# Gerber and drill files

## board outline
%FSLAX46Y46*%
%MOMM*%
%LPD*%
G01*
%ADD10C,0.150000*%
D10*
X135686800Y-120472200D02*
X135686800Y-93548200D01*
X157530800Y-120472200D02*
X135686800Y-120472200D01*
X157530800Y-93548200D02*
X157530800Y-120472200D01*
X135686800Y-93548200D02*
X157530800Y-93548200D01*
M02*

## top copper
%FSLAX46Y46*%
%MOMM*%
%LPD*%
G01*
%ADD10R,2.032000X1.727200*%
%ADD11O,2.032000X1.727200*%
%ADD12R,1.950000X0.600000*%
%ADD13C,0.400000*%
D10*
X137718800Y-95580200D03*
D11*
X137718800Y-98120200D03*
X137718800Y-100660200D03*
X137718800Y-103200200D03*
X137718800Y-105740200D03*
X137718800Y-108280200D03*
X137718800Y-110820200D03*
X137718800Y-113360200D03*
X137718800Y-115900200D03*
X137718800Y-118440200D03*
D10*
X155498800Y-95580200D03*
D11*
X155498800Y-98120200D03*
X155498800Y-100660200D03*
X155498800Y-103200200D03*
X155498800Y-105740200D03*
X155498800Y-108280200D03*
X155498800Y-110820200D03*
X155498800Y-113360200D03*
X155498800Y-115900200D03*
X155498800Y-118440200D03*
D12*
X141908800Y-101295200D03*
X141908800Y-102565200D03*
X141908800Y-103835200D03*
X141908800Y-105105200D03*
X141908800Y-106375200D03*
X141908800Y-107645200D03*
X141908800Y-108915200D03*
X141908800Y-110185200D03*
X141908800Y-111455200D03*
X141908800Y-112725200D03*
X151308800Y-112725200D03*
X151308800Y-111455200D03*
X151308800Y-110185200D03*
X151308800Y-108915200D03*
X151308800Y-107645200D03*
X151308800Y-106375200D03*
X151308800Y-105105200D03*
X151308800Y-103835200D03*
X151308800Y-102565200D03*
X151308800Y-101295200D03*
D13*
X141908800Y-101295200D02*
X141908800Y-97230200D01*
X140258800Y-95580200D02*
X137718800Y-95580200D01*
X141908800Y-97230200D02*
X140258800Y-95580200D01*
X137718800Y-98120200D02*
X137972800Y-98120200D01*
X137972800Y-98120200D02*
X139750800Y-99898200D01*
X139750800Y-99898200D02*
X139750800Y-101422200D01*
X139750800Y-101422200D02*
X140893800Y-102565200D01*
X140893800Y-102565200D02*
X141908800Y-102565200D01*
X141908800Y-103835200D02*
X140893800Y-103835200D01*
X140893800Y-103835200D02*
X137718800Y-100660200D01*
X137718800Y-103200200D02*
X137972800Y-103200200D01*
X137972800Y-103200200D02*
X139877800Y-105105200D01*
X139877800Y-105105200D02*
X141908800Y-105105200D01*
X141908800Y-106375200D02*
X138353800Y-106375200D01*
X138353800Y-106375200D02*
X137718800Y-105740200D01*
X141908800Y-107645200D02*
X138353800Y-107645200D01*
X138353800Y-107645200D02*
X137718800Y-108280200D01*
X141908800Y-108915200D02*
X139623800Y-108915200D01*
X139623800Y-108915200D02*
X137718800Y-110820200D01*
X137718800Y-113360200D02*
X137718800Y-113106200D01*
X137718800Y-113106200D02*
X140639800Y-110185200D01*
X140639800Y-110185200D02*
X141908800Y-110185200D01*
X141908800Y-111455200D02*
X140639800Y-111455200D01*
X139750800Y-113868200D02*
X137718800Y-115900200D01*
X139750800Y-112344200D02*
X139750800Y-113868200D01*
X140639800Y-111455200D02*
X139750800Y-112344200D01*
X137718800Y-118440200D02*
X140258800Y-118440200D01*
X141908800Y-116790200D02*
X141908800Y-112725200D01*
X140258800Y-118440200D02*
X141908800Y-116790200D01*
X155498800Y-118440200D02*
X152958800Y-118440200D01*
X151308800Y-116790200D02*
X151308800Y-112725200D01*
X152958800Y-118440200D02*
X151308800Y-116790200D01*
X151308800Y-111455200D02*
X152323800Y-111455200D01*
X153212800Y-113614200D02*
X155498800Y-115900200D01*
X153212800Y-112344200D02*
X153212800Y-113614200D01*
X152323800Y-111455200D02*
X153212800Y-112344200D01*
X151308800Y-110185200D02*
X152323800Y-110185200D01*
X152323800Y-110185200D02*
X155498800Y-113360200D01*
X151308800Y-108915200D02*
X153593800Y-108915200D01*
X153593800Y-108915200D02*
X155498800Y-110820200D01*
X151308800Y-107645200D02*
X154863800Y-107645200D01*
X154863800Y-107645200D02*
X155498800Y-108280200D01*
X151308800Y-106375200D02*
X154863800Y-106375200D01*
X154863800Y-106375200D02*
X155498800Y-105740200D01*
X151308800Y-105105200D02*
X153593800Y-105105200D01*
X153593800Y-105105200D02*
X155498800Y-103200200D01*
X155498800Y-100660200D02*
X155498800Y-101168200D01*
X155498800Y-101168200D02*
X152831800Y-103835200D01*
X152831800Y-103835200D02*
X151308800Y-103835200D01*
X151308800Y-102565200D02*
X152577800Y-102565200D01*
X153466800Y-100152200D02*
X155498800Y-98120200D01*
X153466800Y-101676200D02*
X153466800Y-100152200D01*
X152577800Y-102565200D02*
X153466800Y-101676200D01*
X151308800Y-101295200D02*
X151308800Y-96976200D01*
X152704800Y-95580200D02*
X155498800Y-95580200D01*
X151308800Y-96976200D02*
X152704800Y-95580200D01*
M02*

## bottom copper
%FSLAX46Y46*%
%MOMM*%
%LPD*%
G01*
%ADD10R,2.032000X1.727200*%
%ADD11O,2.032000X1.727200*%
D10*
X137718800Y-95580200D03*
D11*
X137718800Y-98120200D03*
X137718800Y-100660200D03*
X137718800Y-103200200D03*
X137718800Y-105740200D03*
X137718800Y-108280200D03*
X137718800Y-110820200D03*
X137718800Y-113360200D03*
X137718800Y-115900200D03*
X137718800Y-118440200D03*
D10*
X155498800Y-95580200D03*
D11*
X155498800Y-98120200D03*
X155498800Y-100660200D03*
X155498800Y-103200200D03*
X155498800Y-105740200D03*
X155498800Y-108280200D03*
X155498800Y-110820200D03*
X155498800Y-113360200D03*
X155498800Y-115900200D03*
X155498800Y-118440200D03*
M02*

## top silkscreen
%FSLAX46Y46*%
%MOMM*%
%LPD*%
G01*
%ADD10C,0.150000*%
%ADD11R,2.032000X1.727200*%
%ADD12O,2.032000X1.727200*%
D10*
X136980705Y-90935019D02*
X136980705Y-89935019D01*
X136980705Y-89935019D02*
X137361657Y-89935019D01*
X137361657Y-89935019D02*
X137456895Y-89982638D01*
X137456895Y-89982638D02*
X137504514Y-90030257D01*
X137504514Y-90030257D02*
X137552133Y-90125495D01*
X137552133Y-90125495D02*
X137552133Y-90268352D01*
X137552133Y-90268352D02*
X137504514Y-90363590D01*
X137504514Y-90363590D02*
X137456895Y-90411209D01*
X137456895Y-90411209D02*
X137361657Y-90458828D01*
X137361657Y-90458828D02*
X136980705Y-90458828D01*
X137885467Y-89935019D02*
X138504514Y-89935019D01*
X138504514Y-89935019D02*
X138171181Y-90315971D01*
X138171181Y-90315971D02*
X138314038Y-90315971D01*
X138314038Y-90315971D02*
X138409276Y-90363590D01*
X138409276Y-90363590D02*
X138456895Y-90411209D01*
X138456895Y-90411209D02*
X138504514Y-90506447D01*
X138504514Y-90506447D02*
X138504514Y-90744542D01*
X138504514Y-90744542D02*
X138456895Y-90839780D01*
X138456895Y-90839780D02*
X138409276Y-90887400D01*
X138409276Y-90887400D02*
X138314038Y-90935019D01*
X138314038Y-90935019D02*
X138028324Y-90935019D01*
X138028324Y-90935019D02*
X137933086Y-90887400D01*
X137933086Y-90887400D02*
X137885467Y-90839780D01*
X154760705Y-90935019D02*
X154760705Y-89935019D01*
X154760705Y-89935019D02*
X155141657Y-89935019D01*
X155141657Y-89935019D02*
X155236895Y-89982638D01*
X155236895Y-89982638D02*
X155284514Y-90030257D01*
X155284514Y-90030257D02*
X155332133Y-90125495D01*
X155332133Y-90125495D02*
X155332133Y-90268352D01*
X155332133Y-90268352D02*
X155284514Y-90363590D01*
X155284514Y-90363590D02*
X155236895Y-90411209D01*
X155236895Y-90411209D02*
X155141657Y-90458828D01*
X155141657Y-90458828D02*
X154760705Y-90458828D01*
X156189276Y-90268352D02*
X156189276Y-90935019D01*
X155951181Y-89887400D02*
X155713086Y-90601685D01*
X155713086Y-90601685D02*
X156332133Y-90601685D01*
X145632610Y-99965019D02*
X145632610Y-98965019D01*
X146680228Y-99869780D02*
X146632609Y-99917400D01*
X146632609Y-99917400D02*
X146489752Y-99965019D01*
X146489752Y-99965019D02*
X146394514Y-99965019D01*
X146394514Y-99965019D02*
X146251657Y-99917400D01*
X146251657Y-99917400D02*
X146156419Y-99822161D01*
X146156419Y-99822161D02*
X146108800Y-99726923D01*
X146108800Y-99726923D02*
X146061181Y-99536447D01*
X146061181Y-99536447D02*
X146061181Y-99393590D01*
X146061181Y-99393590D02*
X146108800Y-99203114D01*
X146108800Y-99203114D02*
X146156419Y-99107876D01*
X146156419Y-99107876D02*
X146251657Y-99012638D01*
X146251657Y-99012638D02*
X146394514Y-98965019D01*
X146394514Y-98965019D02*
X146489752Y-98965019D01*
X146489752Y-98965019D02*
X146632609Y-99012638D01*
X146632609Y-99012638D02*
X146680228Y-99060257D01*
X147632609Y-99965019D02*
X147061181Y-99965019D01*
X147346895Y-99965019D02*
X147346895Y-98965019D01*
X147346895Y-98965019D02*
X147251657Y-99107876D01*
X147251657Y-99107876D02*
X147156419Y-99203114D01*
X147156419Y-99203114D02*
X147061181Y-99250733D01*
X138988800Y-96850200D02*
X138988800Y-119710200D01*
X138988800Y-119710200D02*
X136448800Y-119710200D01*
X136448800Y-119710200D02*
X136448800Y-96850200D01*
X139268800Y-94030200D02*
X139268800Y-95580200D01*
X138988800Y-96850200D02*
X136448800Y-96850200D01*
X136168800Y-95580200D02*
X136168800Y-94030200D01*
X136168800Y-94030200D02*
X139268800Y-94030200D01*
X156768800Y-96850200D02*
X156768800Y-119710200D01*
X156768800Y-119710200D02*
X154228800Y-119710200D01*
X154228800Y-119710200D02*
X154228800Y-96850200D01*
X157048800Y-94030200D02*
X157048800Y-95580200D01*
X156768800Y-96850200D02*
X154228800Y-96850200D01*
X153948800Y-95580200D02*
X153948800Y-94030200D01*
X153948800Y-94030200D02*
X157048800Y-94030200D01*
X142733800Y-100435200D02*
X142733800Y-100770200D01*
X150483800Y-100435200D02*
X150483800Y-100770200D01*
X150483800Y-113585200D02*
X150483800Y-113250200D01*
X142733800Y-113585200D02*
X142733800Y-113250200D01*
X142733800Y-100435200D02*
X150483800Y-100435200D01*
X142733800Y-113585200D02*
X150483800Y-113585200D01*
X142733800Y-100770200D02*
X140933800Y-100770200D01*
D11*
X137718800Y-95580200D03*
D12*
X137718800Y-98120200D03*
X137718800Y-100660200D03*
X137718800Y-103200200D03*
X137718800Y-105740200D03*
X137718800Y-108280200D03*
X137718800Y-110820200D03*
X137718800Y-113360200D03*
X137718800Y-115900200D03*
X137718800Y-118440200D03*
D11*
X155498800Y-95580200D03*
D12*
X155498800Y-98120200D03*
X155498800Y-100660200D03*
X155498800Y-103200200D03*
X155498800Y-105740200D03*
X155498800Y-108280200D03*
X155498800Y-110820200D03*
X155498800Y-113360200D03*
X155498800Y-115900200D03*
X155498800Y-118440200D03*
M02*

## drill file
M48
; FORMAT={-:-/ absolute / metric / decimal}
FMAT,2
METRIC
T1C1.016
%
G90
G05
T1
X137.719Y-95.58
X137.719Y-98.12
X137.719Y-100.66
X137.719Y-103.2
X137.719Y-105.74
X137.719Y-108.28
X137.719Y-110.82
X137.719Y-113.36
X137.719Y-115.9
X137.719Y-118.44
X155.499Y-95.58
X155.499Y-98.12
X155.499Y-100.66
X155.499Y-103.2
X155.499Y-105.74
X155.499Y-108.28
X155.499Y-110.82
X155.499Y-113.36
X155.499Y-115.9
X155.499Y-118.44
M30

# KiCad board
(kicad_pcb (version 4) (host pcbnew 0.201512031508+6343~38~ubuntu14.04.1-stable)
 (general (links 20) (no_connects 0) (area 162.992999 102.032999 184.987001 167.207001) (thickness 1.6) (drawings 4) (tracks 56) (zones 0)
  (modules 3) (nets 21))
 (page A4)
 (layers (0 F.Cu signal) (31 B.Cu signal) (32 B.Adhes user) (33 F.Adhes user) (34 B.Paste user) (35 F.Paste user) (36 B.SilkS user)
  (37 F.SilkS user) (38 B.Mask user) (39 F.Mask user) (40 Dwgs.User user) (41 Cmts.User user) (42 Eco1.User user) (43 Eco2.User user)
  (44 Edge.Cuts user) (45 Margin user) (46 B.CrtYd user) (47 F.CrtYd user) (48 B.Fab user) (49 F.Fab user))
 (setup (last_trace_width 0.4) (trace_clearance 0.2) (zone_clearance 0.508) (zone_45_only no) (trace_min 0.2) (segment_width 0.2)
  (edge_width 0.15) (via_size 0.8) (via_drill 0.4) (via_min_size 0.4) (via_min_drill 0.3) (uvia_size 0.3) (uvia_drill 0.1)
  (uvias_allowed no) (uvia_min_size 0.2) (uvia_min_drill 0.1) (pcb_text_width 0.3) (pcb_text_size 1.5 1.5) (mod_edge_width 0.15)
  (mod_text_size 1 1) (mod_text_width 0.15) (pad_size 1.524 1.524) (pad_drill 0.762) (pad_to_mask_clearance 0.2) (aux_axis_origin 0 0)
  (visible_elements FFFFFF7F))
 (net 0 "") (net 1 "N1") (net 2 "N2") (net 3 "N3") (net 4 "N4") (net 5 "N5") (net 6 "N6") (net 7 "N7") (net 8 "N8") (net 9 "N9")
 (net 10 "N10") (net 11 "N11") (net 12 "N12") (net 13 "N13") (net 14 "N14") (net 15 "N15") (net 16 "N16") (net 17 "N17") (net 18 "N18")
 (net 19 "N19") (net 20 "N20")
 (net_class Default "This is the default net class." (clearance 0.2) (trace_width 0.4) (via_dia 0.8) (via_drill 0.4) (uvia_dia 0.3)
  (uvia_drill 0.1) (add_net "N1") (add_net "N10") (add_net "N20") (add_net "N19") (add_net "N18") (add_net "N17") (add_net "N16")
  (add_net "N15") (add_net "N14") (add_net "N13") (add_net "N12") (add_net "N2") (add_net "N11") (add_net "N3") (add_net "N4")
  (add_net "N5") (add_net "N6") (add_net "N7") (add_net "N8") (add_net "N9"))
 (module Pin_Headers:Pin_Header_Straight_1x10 (layer F.Cu) (at 137.7188 95.5802)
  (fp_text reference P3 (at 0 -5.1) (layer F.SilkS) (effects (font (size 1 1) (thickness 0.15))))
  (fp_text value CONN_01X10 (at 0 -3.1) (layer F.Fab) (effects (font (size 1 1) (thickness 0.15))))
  (fp_line (start 1.27 1.27) (end 1.27 24.13) (layer F.SilkS) (width 0.15))
  (fp_line (start 1.27 24.13) (end -1.27 24.13) (layer F.SilkS) (width 0.15))
  (fp_line (start -1.27 24.13) (end -1.27 1.27) (layer F.SilkS) (width 0.15))
  (fp_line (start 1.55 -1.55) (end 1.55 0) (layer F.SilkS) (width 0.15))
  (fp_line (start 1.27 1.27) (end -1.27 1.27) (layer F.SilkS) (width 0.15))
  (fp_line (start -1.55 0) (end -1.55 -1.55) (layer F.SilkS) (width 0.15))
  (fp_line (start -1.55 -1.55) (end 1.55 -1.55) (layer F.SilkS) (width 0.15))
  (pad 1 thru_hole rect (at 0 0) (size 2.032 1.7272) (drill 1.016) (layers *.Cu *.Mask F.SilkS) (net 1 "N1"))
  (pad 2 thru_hole oval (at 0 2.54) (size 2.032 1.7272) (drill 1.016) (layers *.Cu *.Mask F.SilkS) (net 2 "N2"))
  (pad 3 thru_hole oval (at 0 5.08) (size 2.032 1.7272) (drill 1.016) (layers *.Cu *.Mask F.SilkS) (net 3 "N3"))
  (pad 4 thru_hole oval (at 0 7.62) (size 2.032 1.7272) (drill 1.016) (layers *.Cu *.Mask F.SilkS) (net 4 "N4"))
  (pad 5 thru_hole oval (at 0 10.16) (size 2.032 1.7272) (drill 1.016) (layers *.Cu *.Mask F.SilkS) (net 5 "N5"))
  (pad 6 thru_hole oval (at 0 12.7) (size 2.032 1.7272) (drill 1.016) (layers *.Cu *.Mask F.SilkS) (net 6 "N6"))
  (pad 7 thru_hole oval (at 0 15.24) (size 2.032 1.7272) (drill 1.016) (layers *.Cu *.Mask F.SilkS) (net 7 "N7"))
  (pad 8 thru_hole oval (at 0 17.78) (size 2.032 1.7272) (drill 1.016) (layers *.Cu *.Mask F.SilkS) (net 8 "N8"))
  (pad 9 thru_hole oval (at 0 20.32) (size 2.032 1.7272) (drill 1.016) (layers *.Cu *.Mask F.SilkS) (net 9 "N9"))
  (pad 10 thru_hole oval (at 0 22.86) (size 2.032 1.7272) (drill 1.016) (layers *.Cu *.Mask F.SilkS) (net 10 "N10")))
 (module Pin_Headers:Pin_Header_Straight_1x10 (layer F.Cu) (at 155.4988 95.5802)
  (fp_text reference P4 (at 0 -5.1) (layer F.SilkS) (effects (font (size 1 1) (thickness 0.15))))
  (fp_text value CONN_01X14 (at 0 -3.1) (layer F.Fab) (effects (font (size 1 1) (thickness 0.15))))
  (fp_line (start 1.27 1.27) (end 1.27 24.13) (layer F.SilkS) (width 0.15))
  (fp_line (start 1.27 24.13) (end -1.27 24.13) (layer F.SilkS) (width 0.15))
  (fp_line (start -1.27 24.13) (end -1.27 1.27) (layer F.SilkS) (width 0.15))
  (fp_line (start 1.55 -1.55) (end 1.55 0) (layer F.SilkS) (width 0.15))
  (fp_line (start 1.27 1.27) (end -1.27 1.27) (layer F.SilkS) (width 0.15))
  (fp_line (start -1.55 0) (end -1.55 -1.55) (layer F.SilkS) (width 0.15))
  (fp_line (start -1.55 -1.55) (end 1.55 -1.55) (layer F.SilkS) (width 0.15))
  (pad 1 thru_hole rect (at 0 0) (size 2.032 1.7272) (drill 1.016) (layers *.Cu *.Mask F.SilkS) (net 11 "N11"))
  (pad 2 thru_hole oval (at 0 2.54) (size 2.032 1.7272) (drill 1.016) (layers *.Cu *.Mask F.SilkS) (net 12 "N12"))
  (pad 3 thru_hole oval (at 0 5.08) (size 2.032 1.7272) (drill 1.016) (layers *.Cu *.Mask F.SilkS) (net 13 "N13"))
  (pad 4 thru_hole oval (at 0 7.62) (size 2.032 1.7272) (drill 1.016) (layers *.Cu *.Mask F.SilkS) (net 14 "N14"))
  (pad 5 thru_hole oval (at 0 10.16) (size 2.032 1.7272) (drill 1.016) (layers *.Cu *.Mask F.SilkS) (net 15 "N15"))
  (pad 6 thru_hole oval (at 0 12.7) (size 2.032 1.7272) (drill 1.016) (layers *.Cu *.Mask F.SilkS) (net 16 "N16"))
  (pad 7 thru_hole oval (at 0 15.24) (size 2.032 1.7272) (drill 1.016) (layers *.Cu *.Mask F.SilkS) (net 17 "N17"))
  (pad 8 thru_hole oval (at 0 17.78) (size 2.032 1.7272) (drill 1.016) (layers *.Cu *.Mask F.SilkS) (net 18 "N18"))
  (pad 9 thru_hole oval (at 0 20.32) (size 2.032 1.7272) (drill 1.016) (layers *.Cu *.Mask F.SilkS) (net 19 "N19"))
  (pad 10 thru_hole oval (at 0 22.86) (size 2.032 1.7272) (drill 1.016) (layers *.Cu *.Mask F.SilkS) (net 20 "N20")))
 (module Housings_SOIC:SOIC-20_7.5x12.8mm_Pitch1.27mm (layer F.Cu) (at 146.6088 107.0102)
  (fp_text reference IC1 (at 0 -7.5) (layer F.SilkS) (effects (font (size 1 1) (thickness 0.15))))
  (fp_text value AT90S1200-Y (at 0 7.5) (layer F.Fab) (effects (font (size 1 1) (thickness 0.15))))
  (fp_line (start -3.875 -6.575) (end -3.875 -6.24) (layer F.SilkS) (width 0.15))
  (fp_line (start 3.875 -6.575) (end 3.875 -6.24) (layer F.SilkS) (width 0.15))
  (fp_line (start 3.875 6.575) (end 3.875 6.24) (layer F.SilkS) (width 0.15))
  (fp_line (start -3.875 6.575) (end -3.875 6.24) (layer F.SilkS) (width 0.15))
  (fp_line (start -3.875 -6.575) (end 3.875 -6.575) (layer F.SilkS) (width 0.15))
  (fp_line (start -3.875 6.575) (end 3.875 6.575) (layer F.SilkS) (width 0.15))
  (fp_line (start -3.875 -6.24) (end -5.675 -6.24) (layer F.SilkS) (width 0.15))
  (pad 1 smd rect (at -4.7 -5.715) (size 1.95 0.6) (layers F.Cu F.Paste F.Mask) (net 1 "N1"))
  (pad 2 smd rect (at -4.7 -4.445) (size 1.95 0.6) (layers F.Cu F.Paste F.Mask) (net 2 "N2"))
  (pad 3 smd rect (at -4.7 -3.175) (size 1.95 0.6) (layers F.Cu F.Paste F.Mask) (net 3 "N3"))
  (pad 4 smd rect (at -4.7 -1.905) (size 1.95 0.6) (layers F.Cu F.Paste F.Mask) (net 4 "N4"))
  (pad 5 smd rect (at -4.7 -0.635) (size 1.95 0.6) (layers F.Cu F.Paste F.Mask) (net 5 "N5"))
  (pad 6 smd rect (at -4.7 0.635) (size 1.95 0.6) (layers F.Cu F.Paste F.Mask) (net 6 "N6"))
  (pad 7 smd rect (at -4.7 1.905) (size 1.95 0.6) (layers F.Cu F.Paste F.Mask) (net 7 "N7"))
  (pad 8 smd rect (at -4.7 3.175) (size 1.95 0.6) (layers F.Cu F.Paste F.Mask) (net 8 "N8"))
  (pad 9 smd rect (at -4.7 4.445) (size 1.95 0.6) (layers F.Cu F.Paste F.Mask) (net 9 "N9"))
  (pad 10 smd rect (at -4.7 5.715) (size 1.95 0.6) (layers F.Cu F.Paste F.Mask) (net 10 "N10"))
  (pad 11 smd rect (at 4.7 5.715) (size 1.95 0.6) (layers F.Cu F.Paste F.Mask) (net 20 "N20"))
  (pad 12 smd rect (at 4.7 4.445) (size 1.95 0.6) (layers F.Cu F.Paste F.Mask) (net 19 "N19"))
  (pad 13 smd rect (at 4.7 3.175) (size 1.95 0.6) (layers F.Cu F.Paste F.Mask) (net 18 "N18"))
  (pad 14 smd rect (at 4.7 1.905) (size 1.95 0.6) (layers F.Cu F.Paste F.Mask) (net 17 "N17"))
  (pad 15 smd rect (at 4.7 0.635) (size 1.95 0.6) (layers F.Cu F.Paste F.Mask) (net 16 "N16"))
  (pad 16 smd rect (at 4.7 -0.635) (size 1.95 0.6) (layers F.Cu F.Paste F.Mask) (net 15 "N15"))
  (pad 17 smd rect (at 4.7 -1.905) (size 1.95 0.6) (layers F.Cu F.Paste F.Mask) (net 14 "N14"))
  (pad 18 smd rect (at 4.7 -3.175) (size 1.95 0.6) (layers F.Cu F.Paste F.Mask) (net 13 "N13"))
  (pad 19 smd rect (at 4.7 -4.445) (size 1.95 0.6) (layers F.Cu F.Paste F.Mask) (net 12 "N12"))
  (pad 20 smd rect (at 4.7 -5.715) (size 1.95 0.6) (layers F.Cu F.Paste F.Mask) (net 11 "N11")))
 (gr_line (start 135.6868 120.4722) (end 135.6868 93.5482) (angle 90) (layer Edge.Cuts) (width 0.15))
 (gr_line (start 157.5308 120.4722) (end 135.6868 120.4722) (angle 90) (layer Edge.Cuts) (width 0.15))
 (gr_line (start 157.5308 93.5482) (end 157.5308 120.4722) (angle 90) (layer Edge.Cuts) (width 0.15))
 (gr_line (start 135.6868 93.5482) (end 157.5308 93.5482) (angle 90) (layer Edge.Cuts) (width 0.15))
 (segment (start 141.9088 101.2952) (end 141.9088 97.2302) (width 0.4) (layer F.Cu) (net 1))
 (segment (start 140.2588 95.5802) (end 137.7188 95.5802) (width 0.4) (layer F.Cu) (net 1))
 (segment (start 141.9088 97.2302) (end 140.2588 95.5802) (width 0.4) (layer F.Cu) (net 1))
 (segment (start 137.7188 98.1202) (end 137.9728 98.1202) (width 0.4) (layer F.Cu) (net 2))
 (segment (start 137.9728 98.1202) (end 139.7508 99.8982) (width 0.4) (layer F.Cu) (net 2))
 (segment (start 139.7508 99.8982) (end 139.7508 101.4222) (width 0.4) (layer F.Cu) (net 2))
 (segment (start 139.7508 101.4222) (end 140.8938 102.5652) (width 0.4) (layer F.Cu) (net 2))
 (segment (start 140.8938 102.5652) (end 141.9088 102.5652) (width 0.4) (layer F.Cu) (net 2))
 (segment (start 141.9088 103.8352) (end 140.8938 103.8352) (width 0.4) (layer F.Cu) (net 3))
 (segment (start 140.8938 103.8352) (end 137.7188 100.6602) (width 0.4) (layer F.Cu) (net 3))
 (segment (start 137.7188 103.2002) (end 137.9728 103.2002) (width 0.4) (layer F.Cu) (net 4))
 (segment (start 137.9728 103.2002) (end 139.8778 105.1052) (width 0.4) (layer F.Cu) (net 4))
 (segment (start 139.8778 105.1052) (end 141.9088 105.1052) (width 0.4) (layer F.Cu) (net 4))
 (segment (start 141.9088 106.3752) (end 138.3538 106.3752) (width 0.4) (layer F.Cu) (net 5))
 (segment (start 138.3538 106.3752) (end 137.7188 105.7402) (width 0.4) (layer F.Cu) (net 5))
 (segment (start 141.9088 107.6452) (end 138.3538 107.6452) (width 0.4) (layer F.Cu) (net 6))
 (segment (start 138.3538 107.6452) (end 137.7188 108.2802) (width 0.4) (layer F.Cu) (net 6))
 (segment (start 141.9088 108.9152) (end 139.6238 108.9152) (width 0.4) (layer F.Cu) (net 7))
 (segment (start 139.6238 108.9152) (end 137.7188 110.8202) (width 0.4) (layer F.Cu) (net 7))
 (segment (start 137.7188 113.3602) (end 137.7188 113.1062) (width 0.4) (layer F.Cu) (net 8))
 (segment (start 137.7188 113.1062) (end 140.6398 110.1852) (width 0.4) (layer F.Cu) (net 8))
 (segment (start 140.6398 110.1852) (end 141.9088 110.1852) (width 0.4) (layer F.Cu) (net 8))
 (segment (start 141.9088 111.4552) (end 140.6398 111.4552) (width 0.4) (layer F.Cu) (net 9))
 (segment (start 139.7508 113.8682) (end 137.7188 115.9002) (width 0.4) (layer F.Cu) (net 9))
 (segment (start 139.7508 112.3442) (end 139.7508 113.8682) (width 0.4) (layer F.Cu) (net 9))
 (segment (start 140.6398 111.4552) (end 139.7508 112.3442) (width 0.4) (layer F.Cu) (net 9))
 (segment (start 137.7188 118.4402) (end 140.2588 118.4402) (width 0.4) (layer F.Cu) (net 10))
 (segment (start 141.9088 116.7902) (end 141.9088 112.7252) (width 0.4) (layer F.Cu) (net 10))
 (segment (start 140.2588 118.4402) (end 141.9088 116.7902) (width 0.4) (layer F.Cu) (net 10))
 (segment (start 155.4988 118.4402) (end 152.9588 118.4402) (width 0.4) (layer F.Cu) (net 20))
 (segment (start 151.3088 116.7902) (end 151.3088 112.7252) (width 0.4) (layer F.Cu) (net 20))
 (segment (start 152.9588 118.4402) (end 151.3088 116.7902) (width 0.4) (layer F.Cu) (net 20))
 (segment (start 151.3088 111.4552) (end 152.3238 111.4552) (width 0.4) (layer F.Cu) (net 19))
 (segment (start 153.2128 113.6142) (end 155.4988 115.9002) (width 0.4) (layer F.Cu) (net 19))
 (segment (start 153.2128 112.3442) (end 153.2128 113.6142) (width 0.4) (layer F.Cu) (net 19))
 (segment (start 152.3238 111.4552) (end 153.2128 112.3442) (width 0.4) (layer F.Cu) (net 19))
 (segment (start 151.3088 110.1852) (end 152.3238 110.1852) (width 0.4) (layer F.Cu) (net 18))
 (segment (start 152.3238 110.1852) (end 155.4988 113.3602) (width 0.4) (layer F.Cu) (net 18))
 (segment (start 151.3088 108.9152) (end 153.5938 108.9152) (width 0.4) (layer F.Cu) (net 17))
 (segment (start 153.5938 108.9152) (end 155.4988 110.8202) (width 0.4) (layer F.Cu) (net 17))
 (segment (start 151.3088 107.6452) (end 154.8638 107.6452) (width 0.4) (layer F.Cu) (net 16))
 (segment (start 154.8638 107.6452) (end 155.4988 108.2802) (width 0.4) (layer F.Cu) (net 16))
 (segment (start 151.3088 106.3752) (end 154.8638 106.3752) (width 0.4) (layer F.Cu) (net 15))
 (segment (start 154.8638 106.3752) (end 155.4988 105.7402) (width 0.4) (layer F.Cu) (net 15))
 (segment (start 151.3088 105.1052) (end 153.5938 105.1052) (width 0.4) (layer F.Cu) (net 14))
 (segment (start 153.5938 105.1052) (end 155.4988 103.2002) (width 0.4) (layer F.Cu) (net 14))
 (segment (start 155.4988 100.6602) (end 155.4988 101.1682) (width 0.4) (layer F.Cu) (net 13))
 (segment (start 155.4988 101.1682) (end 152.8318 103.8352) (width 0.4) (layer F.Cu) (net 13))
 (segment (start 152.8318 103.8352) (end 151.3088 103.8352) (width 0.4) (layer F.Cu) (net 13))
 (segment (start 151.3088 102.5652) (end 152.5778 102.5652) (width 0.4) (layer F.Cu) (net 12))
 (segment (start 153.4668 100.1522) (end 155.4988 98.1202) (width 0.4) (layer F.Cu) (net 12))
 (segment (start 153.4668 101.6762) (end 153.4668 100.1522) (width 0.4) (layer F.Cu) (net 12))
 (segment (start 152.5778 102.5652) (end 153.4668 101.6762) (width 0.4) (layer F.Cu) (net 12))
 (segment (start 151.3088 101.2952) (end 151.3088 96.9762) (width 0.4) (layer F.Cu) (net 11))
 (segment (start 152.7048 95.5802) (end 155.4988 95.5802) (width 0.4) (layer F.Cu) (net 11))
 (segment (start 151.3088 96.9762) (end 152.7048 95.5802) (width 0.4) (layer F.Cu) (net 11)))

